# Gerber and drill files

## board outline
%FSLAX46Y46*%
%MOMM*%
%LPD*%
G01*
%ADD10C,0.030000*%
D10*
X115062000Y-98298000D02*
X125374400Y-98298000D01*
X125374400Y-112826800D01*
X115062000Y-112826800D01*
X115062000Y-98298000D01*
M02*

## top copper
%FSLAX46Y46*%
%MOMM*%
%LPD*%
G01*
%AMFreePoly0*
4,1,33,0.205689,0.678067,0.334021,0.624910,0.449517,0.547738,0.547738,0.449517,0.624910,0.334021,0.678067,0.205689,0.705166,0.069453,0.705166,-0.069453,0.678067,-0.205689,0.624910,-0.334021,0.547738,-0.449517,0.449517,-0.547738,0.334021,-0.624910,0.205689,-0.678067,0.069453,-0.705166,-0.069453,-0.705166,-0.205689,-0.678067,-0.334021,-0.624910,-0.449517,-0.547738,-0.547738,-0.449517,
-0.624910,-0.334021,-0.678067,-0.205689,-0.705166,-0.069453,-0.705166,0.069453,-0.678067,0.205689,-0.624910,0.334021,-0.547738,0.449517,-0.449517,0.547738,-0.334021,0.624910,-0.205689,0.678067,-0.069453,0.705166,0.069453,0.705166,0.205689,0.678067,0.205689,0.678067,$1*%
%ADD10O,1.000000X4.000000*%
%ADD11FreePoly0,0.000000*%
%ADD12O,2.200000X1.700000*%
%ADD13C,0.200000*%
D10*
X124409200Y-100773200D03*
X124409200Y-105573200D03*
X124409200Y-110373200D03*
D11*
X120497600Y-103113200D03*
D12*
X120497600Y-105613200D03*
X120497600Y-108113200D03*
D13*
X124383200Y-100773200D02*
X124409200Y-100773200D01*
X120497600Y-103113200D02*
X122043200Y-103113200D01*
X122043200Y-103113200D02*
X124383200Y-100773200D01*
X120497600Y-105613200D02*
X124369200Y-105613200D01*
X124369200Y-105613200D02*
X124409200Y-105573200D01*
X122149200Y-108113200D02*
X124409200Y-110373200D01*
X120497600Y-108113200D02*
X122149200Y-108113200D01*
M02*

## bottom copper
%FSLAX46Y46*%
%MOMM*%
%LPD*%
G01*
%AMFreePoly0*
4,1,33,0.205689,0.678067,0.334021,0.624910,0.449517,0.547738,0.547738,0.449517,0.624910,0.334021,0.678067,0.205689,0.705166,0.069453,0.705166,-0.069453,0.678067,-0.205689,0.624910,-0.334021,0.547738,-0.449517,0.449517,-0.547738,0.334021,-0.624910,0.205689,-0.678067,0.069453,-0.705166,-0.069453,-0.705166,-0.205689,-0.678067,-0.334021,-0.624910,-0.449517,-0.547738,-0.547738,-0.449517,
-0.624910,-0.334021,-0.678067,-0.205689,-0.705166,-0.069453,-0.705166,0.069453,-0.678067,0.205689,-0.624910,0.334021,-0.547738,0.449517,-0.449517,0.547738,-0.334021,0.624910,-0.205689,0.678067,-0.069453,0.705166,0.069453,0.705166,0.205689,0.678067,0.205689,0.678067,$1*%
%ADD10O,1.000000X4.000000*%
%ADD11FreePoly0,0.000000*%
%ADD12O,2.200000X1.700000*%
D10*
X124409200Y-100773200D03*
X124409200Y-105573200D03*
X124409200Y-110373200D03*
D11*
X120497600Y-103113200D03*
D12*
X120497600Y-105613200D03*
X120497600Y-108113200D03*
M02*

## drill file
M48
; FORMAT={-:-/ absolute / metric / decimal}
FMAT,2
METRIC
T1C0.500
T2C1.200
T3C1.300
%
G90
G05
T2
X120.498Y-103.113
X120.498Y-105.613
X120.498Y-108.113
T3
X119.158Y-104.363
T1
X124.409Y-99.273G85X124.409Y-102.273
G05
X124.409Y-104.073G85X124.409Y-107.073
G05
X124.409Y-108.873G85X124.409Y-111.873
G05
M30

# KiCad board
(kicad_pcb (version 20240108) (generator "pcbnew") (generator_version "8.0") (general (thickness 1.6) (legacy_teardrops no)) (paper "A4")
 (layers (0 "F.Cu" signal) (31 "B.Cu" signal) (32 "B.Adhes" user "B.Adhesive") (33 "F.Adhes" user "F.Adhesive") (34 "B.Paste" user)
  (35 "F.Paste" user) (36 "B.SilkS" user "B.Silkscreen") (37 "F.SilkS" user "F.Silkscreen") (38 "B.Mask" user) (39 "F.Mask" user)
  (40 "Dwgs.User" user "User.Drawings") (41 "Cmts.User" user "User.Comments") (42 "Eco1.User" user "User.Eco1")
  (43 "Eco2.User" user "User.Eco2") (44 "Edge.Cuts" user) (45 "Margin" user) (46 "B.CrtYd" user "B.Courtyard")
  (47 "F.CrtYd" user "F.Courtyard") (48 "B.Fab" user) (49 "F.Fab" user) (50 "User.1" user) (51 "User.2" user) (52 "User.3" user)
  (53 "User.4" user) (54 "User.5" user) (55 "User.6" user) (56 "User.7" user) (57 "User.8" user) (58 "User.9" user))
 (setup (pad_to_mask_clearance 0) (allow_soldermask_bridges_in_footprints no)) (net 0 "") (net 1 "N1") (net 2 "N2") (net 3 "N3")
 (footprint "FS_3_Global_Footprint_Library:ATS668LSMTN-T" (layer "F.Cu") (at 124.4092 105.5732 -90)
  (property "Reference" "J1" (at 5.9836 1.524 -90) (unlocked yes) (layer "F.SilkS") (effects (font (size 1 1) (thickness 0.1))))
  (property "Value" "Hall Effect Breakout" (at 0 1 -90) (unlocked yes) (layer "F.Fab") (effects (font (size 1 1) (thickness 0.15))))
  (pad "1" thru_hole oval (at -4.8 0 270) (size 4 1) (drill oval 3.5 0.5) (layers "*.Cu" "*.Mask") (remove_unused_layers no) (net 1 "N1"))
  (pad "2" thru_hole oval (at 0 0 270) (size 4 1) (drill oval 3.5 0.5) (layers "*.Cu" "*.Mask") (remove_unused_layers no) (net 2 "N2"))
  (pad "3" thru_hole oval (at 4.8 0 270) (size 4 1) (drill oval 3.5 0.5) (layers "*.Cu" "*.Mask") (remove_unused_layers no) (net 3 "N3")))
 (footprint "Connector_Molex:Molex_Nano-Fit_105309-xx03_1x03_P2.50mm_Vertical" (layer "F.Cu") (at 120.4976 103.1132)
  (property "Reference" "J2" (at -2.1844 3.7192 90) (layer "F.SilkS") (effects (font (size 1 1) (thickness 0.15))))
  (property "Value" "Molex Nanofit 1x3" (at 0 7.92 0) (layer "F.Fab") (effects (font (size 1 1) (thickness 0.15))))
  (pad "" np_thru_hole circle (at -1.34 1.25) (size 1.3 1.3) (drill 1.3) (layers "*.Cu" "*.Mask"))
  (pad "1" thru_hole custom (at 0 0) (size 1.417157 1.417157) (drill 1.2) (layers "*.Cu" "*.Mask") (remove_unused_layers no) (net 1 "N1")
   (thermal_bridge_angle 90) (options (clearance outline) (anchor circle)) (primitives))
  (pad "2" thru_hole oval (at 0 2.5) (size 2.2 1.7) (drill 1.2) (layers "*.Cu" "*.Mask") (remove_unused_layers no) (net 2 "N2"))
  (pad "3" thru_hole oval (at 0 5) (size 2.2 1.7) (drill 1.2) (layers "*.Cu" "*.Mask") (remove_unused_layers no) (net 3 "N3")))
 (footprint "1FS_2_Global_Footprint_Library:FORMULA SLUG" (layer "F.Cu") (at 120.20498 100.490144)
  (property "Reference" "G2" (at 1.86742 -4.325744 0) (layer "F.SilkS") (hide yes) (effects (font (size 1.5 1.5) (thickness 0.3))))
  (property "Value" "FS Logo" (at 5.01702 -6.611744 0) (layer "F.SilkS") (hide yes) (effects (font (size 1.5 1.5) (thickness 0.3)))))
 (gr_rect (start 115.062 98.298) (end 125.3744 112.8268) (stroke (width 0.03) (type default)) (fill none) (layer "Edge.Cuts"))
 (segment (start 124.3832 100.7732) (end 124.4092 100.7732) (width 0.2) (layer "F.Cu") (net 1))
 (segment (start 120.4976 103.1132) (end 122.0432 103.1132) (width 0.2) (layer "F.Cu") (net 1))
 (segment (start 122.0432 103.1132) (end 124.3832 100.7732) (width 0.2) (layer "F.Cu") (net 1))
 (segment (start 120.4976 105.6132) (end 124.3692 105.6132) (width 0.2) (layer "F.Cu") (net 2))
 (segment (start 124.3692 105.6132) (end 124.4092 105.5732) (width 0.2) (layer "F.Cu") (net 2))
 (segment (start 122.1492 108.1132) (end 124.4092 110.3732) (width 0.2) (layer "F.Cu") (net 3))
 (segment (start 120.4976 108.1132) (end 122.1492 108.1132) (width 0.2) (layer "F.Cu") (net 3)))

